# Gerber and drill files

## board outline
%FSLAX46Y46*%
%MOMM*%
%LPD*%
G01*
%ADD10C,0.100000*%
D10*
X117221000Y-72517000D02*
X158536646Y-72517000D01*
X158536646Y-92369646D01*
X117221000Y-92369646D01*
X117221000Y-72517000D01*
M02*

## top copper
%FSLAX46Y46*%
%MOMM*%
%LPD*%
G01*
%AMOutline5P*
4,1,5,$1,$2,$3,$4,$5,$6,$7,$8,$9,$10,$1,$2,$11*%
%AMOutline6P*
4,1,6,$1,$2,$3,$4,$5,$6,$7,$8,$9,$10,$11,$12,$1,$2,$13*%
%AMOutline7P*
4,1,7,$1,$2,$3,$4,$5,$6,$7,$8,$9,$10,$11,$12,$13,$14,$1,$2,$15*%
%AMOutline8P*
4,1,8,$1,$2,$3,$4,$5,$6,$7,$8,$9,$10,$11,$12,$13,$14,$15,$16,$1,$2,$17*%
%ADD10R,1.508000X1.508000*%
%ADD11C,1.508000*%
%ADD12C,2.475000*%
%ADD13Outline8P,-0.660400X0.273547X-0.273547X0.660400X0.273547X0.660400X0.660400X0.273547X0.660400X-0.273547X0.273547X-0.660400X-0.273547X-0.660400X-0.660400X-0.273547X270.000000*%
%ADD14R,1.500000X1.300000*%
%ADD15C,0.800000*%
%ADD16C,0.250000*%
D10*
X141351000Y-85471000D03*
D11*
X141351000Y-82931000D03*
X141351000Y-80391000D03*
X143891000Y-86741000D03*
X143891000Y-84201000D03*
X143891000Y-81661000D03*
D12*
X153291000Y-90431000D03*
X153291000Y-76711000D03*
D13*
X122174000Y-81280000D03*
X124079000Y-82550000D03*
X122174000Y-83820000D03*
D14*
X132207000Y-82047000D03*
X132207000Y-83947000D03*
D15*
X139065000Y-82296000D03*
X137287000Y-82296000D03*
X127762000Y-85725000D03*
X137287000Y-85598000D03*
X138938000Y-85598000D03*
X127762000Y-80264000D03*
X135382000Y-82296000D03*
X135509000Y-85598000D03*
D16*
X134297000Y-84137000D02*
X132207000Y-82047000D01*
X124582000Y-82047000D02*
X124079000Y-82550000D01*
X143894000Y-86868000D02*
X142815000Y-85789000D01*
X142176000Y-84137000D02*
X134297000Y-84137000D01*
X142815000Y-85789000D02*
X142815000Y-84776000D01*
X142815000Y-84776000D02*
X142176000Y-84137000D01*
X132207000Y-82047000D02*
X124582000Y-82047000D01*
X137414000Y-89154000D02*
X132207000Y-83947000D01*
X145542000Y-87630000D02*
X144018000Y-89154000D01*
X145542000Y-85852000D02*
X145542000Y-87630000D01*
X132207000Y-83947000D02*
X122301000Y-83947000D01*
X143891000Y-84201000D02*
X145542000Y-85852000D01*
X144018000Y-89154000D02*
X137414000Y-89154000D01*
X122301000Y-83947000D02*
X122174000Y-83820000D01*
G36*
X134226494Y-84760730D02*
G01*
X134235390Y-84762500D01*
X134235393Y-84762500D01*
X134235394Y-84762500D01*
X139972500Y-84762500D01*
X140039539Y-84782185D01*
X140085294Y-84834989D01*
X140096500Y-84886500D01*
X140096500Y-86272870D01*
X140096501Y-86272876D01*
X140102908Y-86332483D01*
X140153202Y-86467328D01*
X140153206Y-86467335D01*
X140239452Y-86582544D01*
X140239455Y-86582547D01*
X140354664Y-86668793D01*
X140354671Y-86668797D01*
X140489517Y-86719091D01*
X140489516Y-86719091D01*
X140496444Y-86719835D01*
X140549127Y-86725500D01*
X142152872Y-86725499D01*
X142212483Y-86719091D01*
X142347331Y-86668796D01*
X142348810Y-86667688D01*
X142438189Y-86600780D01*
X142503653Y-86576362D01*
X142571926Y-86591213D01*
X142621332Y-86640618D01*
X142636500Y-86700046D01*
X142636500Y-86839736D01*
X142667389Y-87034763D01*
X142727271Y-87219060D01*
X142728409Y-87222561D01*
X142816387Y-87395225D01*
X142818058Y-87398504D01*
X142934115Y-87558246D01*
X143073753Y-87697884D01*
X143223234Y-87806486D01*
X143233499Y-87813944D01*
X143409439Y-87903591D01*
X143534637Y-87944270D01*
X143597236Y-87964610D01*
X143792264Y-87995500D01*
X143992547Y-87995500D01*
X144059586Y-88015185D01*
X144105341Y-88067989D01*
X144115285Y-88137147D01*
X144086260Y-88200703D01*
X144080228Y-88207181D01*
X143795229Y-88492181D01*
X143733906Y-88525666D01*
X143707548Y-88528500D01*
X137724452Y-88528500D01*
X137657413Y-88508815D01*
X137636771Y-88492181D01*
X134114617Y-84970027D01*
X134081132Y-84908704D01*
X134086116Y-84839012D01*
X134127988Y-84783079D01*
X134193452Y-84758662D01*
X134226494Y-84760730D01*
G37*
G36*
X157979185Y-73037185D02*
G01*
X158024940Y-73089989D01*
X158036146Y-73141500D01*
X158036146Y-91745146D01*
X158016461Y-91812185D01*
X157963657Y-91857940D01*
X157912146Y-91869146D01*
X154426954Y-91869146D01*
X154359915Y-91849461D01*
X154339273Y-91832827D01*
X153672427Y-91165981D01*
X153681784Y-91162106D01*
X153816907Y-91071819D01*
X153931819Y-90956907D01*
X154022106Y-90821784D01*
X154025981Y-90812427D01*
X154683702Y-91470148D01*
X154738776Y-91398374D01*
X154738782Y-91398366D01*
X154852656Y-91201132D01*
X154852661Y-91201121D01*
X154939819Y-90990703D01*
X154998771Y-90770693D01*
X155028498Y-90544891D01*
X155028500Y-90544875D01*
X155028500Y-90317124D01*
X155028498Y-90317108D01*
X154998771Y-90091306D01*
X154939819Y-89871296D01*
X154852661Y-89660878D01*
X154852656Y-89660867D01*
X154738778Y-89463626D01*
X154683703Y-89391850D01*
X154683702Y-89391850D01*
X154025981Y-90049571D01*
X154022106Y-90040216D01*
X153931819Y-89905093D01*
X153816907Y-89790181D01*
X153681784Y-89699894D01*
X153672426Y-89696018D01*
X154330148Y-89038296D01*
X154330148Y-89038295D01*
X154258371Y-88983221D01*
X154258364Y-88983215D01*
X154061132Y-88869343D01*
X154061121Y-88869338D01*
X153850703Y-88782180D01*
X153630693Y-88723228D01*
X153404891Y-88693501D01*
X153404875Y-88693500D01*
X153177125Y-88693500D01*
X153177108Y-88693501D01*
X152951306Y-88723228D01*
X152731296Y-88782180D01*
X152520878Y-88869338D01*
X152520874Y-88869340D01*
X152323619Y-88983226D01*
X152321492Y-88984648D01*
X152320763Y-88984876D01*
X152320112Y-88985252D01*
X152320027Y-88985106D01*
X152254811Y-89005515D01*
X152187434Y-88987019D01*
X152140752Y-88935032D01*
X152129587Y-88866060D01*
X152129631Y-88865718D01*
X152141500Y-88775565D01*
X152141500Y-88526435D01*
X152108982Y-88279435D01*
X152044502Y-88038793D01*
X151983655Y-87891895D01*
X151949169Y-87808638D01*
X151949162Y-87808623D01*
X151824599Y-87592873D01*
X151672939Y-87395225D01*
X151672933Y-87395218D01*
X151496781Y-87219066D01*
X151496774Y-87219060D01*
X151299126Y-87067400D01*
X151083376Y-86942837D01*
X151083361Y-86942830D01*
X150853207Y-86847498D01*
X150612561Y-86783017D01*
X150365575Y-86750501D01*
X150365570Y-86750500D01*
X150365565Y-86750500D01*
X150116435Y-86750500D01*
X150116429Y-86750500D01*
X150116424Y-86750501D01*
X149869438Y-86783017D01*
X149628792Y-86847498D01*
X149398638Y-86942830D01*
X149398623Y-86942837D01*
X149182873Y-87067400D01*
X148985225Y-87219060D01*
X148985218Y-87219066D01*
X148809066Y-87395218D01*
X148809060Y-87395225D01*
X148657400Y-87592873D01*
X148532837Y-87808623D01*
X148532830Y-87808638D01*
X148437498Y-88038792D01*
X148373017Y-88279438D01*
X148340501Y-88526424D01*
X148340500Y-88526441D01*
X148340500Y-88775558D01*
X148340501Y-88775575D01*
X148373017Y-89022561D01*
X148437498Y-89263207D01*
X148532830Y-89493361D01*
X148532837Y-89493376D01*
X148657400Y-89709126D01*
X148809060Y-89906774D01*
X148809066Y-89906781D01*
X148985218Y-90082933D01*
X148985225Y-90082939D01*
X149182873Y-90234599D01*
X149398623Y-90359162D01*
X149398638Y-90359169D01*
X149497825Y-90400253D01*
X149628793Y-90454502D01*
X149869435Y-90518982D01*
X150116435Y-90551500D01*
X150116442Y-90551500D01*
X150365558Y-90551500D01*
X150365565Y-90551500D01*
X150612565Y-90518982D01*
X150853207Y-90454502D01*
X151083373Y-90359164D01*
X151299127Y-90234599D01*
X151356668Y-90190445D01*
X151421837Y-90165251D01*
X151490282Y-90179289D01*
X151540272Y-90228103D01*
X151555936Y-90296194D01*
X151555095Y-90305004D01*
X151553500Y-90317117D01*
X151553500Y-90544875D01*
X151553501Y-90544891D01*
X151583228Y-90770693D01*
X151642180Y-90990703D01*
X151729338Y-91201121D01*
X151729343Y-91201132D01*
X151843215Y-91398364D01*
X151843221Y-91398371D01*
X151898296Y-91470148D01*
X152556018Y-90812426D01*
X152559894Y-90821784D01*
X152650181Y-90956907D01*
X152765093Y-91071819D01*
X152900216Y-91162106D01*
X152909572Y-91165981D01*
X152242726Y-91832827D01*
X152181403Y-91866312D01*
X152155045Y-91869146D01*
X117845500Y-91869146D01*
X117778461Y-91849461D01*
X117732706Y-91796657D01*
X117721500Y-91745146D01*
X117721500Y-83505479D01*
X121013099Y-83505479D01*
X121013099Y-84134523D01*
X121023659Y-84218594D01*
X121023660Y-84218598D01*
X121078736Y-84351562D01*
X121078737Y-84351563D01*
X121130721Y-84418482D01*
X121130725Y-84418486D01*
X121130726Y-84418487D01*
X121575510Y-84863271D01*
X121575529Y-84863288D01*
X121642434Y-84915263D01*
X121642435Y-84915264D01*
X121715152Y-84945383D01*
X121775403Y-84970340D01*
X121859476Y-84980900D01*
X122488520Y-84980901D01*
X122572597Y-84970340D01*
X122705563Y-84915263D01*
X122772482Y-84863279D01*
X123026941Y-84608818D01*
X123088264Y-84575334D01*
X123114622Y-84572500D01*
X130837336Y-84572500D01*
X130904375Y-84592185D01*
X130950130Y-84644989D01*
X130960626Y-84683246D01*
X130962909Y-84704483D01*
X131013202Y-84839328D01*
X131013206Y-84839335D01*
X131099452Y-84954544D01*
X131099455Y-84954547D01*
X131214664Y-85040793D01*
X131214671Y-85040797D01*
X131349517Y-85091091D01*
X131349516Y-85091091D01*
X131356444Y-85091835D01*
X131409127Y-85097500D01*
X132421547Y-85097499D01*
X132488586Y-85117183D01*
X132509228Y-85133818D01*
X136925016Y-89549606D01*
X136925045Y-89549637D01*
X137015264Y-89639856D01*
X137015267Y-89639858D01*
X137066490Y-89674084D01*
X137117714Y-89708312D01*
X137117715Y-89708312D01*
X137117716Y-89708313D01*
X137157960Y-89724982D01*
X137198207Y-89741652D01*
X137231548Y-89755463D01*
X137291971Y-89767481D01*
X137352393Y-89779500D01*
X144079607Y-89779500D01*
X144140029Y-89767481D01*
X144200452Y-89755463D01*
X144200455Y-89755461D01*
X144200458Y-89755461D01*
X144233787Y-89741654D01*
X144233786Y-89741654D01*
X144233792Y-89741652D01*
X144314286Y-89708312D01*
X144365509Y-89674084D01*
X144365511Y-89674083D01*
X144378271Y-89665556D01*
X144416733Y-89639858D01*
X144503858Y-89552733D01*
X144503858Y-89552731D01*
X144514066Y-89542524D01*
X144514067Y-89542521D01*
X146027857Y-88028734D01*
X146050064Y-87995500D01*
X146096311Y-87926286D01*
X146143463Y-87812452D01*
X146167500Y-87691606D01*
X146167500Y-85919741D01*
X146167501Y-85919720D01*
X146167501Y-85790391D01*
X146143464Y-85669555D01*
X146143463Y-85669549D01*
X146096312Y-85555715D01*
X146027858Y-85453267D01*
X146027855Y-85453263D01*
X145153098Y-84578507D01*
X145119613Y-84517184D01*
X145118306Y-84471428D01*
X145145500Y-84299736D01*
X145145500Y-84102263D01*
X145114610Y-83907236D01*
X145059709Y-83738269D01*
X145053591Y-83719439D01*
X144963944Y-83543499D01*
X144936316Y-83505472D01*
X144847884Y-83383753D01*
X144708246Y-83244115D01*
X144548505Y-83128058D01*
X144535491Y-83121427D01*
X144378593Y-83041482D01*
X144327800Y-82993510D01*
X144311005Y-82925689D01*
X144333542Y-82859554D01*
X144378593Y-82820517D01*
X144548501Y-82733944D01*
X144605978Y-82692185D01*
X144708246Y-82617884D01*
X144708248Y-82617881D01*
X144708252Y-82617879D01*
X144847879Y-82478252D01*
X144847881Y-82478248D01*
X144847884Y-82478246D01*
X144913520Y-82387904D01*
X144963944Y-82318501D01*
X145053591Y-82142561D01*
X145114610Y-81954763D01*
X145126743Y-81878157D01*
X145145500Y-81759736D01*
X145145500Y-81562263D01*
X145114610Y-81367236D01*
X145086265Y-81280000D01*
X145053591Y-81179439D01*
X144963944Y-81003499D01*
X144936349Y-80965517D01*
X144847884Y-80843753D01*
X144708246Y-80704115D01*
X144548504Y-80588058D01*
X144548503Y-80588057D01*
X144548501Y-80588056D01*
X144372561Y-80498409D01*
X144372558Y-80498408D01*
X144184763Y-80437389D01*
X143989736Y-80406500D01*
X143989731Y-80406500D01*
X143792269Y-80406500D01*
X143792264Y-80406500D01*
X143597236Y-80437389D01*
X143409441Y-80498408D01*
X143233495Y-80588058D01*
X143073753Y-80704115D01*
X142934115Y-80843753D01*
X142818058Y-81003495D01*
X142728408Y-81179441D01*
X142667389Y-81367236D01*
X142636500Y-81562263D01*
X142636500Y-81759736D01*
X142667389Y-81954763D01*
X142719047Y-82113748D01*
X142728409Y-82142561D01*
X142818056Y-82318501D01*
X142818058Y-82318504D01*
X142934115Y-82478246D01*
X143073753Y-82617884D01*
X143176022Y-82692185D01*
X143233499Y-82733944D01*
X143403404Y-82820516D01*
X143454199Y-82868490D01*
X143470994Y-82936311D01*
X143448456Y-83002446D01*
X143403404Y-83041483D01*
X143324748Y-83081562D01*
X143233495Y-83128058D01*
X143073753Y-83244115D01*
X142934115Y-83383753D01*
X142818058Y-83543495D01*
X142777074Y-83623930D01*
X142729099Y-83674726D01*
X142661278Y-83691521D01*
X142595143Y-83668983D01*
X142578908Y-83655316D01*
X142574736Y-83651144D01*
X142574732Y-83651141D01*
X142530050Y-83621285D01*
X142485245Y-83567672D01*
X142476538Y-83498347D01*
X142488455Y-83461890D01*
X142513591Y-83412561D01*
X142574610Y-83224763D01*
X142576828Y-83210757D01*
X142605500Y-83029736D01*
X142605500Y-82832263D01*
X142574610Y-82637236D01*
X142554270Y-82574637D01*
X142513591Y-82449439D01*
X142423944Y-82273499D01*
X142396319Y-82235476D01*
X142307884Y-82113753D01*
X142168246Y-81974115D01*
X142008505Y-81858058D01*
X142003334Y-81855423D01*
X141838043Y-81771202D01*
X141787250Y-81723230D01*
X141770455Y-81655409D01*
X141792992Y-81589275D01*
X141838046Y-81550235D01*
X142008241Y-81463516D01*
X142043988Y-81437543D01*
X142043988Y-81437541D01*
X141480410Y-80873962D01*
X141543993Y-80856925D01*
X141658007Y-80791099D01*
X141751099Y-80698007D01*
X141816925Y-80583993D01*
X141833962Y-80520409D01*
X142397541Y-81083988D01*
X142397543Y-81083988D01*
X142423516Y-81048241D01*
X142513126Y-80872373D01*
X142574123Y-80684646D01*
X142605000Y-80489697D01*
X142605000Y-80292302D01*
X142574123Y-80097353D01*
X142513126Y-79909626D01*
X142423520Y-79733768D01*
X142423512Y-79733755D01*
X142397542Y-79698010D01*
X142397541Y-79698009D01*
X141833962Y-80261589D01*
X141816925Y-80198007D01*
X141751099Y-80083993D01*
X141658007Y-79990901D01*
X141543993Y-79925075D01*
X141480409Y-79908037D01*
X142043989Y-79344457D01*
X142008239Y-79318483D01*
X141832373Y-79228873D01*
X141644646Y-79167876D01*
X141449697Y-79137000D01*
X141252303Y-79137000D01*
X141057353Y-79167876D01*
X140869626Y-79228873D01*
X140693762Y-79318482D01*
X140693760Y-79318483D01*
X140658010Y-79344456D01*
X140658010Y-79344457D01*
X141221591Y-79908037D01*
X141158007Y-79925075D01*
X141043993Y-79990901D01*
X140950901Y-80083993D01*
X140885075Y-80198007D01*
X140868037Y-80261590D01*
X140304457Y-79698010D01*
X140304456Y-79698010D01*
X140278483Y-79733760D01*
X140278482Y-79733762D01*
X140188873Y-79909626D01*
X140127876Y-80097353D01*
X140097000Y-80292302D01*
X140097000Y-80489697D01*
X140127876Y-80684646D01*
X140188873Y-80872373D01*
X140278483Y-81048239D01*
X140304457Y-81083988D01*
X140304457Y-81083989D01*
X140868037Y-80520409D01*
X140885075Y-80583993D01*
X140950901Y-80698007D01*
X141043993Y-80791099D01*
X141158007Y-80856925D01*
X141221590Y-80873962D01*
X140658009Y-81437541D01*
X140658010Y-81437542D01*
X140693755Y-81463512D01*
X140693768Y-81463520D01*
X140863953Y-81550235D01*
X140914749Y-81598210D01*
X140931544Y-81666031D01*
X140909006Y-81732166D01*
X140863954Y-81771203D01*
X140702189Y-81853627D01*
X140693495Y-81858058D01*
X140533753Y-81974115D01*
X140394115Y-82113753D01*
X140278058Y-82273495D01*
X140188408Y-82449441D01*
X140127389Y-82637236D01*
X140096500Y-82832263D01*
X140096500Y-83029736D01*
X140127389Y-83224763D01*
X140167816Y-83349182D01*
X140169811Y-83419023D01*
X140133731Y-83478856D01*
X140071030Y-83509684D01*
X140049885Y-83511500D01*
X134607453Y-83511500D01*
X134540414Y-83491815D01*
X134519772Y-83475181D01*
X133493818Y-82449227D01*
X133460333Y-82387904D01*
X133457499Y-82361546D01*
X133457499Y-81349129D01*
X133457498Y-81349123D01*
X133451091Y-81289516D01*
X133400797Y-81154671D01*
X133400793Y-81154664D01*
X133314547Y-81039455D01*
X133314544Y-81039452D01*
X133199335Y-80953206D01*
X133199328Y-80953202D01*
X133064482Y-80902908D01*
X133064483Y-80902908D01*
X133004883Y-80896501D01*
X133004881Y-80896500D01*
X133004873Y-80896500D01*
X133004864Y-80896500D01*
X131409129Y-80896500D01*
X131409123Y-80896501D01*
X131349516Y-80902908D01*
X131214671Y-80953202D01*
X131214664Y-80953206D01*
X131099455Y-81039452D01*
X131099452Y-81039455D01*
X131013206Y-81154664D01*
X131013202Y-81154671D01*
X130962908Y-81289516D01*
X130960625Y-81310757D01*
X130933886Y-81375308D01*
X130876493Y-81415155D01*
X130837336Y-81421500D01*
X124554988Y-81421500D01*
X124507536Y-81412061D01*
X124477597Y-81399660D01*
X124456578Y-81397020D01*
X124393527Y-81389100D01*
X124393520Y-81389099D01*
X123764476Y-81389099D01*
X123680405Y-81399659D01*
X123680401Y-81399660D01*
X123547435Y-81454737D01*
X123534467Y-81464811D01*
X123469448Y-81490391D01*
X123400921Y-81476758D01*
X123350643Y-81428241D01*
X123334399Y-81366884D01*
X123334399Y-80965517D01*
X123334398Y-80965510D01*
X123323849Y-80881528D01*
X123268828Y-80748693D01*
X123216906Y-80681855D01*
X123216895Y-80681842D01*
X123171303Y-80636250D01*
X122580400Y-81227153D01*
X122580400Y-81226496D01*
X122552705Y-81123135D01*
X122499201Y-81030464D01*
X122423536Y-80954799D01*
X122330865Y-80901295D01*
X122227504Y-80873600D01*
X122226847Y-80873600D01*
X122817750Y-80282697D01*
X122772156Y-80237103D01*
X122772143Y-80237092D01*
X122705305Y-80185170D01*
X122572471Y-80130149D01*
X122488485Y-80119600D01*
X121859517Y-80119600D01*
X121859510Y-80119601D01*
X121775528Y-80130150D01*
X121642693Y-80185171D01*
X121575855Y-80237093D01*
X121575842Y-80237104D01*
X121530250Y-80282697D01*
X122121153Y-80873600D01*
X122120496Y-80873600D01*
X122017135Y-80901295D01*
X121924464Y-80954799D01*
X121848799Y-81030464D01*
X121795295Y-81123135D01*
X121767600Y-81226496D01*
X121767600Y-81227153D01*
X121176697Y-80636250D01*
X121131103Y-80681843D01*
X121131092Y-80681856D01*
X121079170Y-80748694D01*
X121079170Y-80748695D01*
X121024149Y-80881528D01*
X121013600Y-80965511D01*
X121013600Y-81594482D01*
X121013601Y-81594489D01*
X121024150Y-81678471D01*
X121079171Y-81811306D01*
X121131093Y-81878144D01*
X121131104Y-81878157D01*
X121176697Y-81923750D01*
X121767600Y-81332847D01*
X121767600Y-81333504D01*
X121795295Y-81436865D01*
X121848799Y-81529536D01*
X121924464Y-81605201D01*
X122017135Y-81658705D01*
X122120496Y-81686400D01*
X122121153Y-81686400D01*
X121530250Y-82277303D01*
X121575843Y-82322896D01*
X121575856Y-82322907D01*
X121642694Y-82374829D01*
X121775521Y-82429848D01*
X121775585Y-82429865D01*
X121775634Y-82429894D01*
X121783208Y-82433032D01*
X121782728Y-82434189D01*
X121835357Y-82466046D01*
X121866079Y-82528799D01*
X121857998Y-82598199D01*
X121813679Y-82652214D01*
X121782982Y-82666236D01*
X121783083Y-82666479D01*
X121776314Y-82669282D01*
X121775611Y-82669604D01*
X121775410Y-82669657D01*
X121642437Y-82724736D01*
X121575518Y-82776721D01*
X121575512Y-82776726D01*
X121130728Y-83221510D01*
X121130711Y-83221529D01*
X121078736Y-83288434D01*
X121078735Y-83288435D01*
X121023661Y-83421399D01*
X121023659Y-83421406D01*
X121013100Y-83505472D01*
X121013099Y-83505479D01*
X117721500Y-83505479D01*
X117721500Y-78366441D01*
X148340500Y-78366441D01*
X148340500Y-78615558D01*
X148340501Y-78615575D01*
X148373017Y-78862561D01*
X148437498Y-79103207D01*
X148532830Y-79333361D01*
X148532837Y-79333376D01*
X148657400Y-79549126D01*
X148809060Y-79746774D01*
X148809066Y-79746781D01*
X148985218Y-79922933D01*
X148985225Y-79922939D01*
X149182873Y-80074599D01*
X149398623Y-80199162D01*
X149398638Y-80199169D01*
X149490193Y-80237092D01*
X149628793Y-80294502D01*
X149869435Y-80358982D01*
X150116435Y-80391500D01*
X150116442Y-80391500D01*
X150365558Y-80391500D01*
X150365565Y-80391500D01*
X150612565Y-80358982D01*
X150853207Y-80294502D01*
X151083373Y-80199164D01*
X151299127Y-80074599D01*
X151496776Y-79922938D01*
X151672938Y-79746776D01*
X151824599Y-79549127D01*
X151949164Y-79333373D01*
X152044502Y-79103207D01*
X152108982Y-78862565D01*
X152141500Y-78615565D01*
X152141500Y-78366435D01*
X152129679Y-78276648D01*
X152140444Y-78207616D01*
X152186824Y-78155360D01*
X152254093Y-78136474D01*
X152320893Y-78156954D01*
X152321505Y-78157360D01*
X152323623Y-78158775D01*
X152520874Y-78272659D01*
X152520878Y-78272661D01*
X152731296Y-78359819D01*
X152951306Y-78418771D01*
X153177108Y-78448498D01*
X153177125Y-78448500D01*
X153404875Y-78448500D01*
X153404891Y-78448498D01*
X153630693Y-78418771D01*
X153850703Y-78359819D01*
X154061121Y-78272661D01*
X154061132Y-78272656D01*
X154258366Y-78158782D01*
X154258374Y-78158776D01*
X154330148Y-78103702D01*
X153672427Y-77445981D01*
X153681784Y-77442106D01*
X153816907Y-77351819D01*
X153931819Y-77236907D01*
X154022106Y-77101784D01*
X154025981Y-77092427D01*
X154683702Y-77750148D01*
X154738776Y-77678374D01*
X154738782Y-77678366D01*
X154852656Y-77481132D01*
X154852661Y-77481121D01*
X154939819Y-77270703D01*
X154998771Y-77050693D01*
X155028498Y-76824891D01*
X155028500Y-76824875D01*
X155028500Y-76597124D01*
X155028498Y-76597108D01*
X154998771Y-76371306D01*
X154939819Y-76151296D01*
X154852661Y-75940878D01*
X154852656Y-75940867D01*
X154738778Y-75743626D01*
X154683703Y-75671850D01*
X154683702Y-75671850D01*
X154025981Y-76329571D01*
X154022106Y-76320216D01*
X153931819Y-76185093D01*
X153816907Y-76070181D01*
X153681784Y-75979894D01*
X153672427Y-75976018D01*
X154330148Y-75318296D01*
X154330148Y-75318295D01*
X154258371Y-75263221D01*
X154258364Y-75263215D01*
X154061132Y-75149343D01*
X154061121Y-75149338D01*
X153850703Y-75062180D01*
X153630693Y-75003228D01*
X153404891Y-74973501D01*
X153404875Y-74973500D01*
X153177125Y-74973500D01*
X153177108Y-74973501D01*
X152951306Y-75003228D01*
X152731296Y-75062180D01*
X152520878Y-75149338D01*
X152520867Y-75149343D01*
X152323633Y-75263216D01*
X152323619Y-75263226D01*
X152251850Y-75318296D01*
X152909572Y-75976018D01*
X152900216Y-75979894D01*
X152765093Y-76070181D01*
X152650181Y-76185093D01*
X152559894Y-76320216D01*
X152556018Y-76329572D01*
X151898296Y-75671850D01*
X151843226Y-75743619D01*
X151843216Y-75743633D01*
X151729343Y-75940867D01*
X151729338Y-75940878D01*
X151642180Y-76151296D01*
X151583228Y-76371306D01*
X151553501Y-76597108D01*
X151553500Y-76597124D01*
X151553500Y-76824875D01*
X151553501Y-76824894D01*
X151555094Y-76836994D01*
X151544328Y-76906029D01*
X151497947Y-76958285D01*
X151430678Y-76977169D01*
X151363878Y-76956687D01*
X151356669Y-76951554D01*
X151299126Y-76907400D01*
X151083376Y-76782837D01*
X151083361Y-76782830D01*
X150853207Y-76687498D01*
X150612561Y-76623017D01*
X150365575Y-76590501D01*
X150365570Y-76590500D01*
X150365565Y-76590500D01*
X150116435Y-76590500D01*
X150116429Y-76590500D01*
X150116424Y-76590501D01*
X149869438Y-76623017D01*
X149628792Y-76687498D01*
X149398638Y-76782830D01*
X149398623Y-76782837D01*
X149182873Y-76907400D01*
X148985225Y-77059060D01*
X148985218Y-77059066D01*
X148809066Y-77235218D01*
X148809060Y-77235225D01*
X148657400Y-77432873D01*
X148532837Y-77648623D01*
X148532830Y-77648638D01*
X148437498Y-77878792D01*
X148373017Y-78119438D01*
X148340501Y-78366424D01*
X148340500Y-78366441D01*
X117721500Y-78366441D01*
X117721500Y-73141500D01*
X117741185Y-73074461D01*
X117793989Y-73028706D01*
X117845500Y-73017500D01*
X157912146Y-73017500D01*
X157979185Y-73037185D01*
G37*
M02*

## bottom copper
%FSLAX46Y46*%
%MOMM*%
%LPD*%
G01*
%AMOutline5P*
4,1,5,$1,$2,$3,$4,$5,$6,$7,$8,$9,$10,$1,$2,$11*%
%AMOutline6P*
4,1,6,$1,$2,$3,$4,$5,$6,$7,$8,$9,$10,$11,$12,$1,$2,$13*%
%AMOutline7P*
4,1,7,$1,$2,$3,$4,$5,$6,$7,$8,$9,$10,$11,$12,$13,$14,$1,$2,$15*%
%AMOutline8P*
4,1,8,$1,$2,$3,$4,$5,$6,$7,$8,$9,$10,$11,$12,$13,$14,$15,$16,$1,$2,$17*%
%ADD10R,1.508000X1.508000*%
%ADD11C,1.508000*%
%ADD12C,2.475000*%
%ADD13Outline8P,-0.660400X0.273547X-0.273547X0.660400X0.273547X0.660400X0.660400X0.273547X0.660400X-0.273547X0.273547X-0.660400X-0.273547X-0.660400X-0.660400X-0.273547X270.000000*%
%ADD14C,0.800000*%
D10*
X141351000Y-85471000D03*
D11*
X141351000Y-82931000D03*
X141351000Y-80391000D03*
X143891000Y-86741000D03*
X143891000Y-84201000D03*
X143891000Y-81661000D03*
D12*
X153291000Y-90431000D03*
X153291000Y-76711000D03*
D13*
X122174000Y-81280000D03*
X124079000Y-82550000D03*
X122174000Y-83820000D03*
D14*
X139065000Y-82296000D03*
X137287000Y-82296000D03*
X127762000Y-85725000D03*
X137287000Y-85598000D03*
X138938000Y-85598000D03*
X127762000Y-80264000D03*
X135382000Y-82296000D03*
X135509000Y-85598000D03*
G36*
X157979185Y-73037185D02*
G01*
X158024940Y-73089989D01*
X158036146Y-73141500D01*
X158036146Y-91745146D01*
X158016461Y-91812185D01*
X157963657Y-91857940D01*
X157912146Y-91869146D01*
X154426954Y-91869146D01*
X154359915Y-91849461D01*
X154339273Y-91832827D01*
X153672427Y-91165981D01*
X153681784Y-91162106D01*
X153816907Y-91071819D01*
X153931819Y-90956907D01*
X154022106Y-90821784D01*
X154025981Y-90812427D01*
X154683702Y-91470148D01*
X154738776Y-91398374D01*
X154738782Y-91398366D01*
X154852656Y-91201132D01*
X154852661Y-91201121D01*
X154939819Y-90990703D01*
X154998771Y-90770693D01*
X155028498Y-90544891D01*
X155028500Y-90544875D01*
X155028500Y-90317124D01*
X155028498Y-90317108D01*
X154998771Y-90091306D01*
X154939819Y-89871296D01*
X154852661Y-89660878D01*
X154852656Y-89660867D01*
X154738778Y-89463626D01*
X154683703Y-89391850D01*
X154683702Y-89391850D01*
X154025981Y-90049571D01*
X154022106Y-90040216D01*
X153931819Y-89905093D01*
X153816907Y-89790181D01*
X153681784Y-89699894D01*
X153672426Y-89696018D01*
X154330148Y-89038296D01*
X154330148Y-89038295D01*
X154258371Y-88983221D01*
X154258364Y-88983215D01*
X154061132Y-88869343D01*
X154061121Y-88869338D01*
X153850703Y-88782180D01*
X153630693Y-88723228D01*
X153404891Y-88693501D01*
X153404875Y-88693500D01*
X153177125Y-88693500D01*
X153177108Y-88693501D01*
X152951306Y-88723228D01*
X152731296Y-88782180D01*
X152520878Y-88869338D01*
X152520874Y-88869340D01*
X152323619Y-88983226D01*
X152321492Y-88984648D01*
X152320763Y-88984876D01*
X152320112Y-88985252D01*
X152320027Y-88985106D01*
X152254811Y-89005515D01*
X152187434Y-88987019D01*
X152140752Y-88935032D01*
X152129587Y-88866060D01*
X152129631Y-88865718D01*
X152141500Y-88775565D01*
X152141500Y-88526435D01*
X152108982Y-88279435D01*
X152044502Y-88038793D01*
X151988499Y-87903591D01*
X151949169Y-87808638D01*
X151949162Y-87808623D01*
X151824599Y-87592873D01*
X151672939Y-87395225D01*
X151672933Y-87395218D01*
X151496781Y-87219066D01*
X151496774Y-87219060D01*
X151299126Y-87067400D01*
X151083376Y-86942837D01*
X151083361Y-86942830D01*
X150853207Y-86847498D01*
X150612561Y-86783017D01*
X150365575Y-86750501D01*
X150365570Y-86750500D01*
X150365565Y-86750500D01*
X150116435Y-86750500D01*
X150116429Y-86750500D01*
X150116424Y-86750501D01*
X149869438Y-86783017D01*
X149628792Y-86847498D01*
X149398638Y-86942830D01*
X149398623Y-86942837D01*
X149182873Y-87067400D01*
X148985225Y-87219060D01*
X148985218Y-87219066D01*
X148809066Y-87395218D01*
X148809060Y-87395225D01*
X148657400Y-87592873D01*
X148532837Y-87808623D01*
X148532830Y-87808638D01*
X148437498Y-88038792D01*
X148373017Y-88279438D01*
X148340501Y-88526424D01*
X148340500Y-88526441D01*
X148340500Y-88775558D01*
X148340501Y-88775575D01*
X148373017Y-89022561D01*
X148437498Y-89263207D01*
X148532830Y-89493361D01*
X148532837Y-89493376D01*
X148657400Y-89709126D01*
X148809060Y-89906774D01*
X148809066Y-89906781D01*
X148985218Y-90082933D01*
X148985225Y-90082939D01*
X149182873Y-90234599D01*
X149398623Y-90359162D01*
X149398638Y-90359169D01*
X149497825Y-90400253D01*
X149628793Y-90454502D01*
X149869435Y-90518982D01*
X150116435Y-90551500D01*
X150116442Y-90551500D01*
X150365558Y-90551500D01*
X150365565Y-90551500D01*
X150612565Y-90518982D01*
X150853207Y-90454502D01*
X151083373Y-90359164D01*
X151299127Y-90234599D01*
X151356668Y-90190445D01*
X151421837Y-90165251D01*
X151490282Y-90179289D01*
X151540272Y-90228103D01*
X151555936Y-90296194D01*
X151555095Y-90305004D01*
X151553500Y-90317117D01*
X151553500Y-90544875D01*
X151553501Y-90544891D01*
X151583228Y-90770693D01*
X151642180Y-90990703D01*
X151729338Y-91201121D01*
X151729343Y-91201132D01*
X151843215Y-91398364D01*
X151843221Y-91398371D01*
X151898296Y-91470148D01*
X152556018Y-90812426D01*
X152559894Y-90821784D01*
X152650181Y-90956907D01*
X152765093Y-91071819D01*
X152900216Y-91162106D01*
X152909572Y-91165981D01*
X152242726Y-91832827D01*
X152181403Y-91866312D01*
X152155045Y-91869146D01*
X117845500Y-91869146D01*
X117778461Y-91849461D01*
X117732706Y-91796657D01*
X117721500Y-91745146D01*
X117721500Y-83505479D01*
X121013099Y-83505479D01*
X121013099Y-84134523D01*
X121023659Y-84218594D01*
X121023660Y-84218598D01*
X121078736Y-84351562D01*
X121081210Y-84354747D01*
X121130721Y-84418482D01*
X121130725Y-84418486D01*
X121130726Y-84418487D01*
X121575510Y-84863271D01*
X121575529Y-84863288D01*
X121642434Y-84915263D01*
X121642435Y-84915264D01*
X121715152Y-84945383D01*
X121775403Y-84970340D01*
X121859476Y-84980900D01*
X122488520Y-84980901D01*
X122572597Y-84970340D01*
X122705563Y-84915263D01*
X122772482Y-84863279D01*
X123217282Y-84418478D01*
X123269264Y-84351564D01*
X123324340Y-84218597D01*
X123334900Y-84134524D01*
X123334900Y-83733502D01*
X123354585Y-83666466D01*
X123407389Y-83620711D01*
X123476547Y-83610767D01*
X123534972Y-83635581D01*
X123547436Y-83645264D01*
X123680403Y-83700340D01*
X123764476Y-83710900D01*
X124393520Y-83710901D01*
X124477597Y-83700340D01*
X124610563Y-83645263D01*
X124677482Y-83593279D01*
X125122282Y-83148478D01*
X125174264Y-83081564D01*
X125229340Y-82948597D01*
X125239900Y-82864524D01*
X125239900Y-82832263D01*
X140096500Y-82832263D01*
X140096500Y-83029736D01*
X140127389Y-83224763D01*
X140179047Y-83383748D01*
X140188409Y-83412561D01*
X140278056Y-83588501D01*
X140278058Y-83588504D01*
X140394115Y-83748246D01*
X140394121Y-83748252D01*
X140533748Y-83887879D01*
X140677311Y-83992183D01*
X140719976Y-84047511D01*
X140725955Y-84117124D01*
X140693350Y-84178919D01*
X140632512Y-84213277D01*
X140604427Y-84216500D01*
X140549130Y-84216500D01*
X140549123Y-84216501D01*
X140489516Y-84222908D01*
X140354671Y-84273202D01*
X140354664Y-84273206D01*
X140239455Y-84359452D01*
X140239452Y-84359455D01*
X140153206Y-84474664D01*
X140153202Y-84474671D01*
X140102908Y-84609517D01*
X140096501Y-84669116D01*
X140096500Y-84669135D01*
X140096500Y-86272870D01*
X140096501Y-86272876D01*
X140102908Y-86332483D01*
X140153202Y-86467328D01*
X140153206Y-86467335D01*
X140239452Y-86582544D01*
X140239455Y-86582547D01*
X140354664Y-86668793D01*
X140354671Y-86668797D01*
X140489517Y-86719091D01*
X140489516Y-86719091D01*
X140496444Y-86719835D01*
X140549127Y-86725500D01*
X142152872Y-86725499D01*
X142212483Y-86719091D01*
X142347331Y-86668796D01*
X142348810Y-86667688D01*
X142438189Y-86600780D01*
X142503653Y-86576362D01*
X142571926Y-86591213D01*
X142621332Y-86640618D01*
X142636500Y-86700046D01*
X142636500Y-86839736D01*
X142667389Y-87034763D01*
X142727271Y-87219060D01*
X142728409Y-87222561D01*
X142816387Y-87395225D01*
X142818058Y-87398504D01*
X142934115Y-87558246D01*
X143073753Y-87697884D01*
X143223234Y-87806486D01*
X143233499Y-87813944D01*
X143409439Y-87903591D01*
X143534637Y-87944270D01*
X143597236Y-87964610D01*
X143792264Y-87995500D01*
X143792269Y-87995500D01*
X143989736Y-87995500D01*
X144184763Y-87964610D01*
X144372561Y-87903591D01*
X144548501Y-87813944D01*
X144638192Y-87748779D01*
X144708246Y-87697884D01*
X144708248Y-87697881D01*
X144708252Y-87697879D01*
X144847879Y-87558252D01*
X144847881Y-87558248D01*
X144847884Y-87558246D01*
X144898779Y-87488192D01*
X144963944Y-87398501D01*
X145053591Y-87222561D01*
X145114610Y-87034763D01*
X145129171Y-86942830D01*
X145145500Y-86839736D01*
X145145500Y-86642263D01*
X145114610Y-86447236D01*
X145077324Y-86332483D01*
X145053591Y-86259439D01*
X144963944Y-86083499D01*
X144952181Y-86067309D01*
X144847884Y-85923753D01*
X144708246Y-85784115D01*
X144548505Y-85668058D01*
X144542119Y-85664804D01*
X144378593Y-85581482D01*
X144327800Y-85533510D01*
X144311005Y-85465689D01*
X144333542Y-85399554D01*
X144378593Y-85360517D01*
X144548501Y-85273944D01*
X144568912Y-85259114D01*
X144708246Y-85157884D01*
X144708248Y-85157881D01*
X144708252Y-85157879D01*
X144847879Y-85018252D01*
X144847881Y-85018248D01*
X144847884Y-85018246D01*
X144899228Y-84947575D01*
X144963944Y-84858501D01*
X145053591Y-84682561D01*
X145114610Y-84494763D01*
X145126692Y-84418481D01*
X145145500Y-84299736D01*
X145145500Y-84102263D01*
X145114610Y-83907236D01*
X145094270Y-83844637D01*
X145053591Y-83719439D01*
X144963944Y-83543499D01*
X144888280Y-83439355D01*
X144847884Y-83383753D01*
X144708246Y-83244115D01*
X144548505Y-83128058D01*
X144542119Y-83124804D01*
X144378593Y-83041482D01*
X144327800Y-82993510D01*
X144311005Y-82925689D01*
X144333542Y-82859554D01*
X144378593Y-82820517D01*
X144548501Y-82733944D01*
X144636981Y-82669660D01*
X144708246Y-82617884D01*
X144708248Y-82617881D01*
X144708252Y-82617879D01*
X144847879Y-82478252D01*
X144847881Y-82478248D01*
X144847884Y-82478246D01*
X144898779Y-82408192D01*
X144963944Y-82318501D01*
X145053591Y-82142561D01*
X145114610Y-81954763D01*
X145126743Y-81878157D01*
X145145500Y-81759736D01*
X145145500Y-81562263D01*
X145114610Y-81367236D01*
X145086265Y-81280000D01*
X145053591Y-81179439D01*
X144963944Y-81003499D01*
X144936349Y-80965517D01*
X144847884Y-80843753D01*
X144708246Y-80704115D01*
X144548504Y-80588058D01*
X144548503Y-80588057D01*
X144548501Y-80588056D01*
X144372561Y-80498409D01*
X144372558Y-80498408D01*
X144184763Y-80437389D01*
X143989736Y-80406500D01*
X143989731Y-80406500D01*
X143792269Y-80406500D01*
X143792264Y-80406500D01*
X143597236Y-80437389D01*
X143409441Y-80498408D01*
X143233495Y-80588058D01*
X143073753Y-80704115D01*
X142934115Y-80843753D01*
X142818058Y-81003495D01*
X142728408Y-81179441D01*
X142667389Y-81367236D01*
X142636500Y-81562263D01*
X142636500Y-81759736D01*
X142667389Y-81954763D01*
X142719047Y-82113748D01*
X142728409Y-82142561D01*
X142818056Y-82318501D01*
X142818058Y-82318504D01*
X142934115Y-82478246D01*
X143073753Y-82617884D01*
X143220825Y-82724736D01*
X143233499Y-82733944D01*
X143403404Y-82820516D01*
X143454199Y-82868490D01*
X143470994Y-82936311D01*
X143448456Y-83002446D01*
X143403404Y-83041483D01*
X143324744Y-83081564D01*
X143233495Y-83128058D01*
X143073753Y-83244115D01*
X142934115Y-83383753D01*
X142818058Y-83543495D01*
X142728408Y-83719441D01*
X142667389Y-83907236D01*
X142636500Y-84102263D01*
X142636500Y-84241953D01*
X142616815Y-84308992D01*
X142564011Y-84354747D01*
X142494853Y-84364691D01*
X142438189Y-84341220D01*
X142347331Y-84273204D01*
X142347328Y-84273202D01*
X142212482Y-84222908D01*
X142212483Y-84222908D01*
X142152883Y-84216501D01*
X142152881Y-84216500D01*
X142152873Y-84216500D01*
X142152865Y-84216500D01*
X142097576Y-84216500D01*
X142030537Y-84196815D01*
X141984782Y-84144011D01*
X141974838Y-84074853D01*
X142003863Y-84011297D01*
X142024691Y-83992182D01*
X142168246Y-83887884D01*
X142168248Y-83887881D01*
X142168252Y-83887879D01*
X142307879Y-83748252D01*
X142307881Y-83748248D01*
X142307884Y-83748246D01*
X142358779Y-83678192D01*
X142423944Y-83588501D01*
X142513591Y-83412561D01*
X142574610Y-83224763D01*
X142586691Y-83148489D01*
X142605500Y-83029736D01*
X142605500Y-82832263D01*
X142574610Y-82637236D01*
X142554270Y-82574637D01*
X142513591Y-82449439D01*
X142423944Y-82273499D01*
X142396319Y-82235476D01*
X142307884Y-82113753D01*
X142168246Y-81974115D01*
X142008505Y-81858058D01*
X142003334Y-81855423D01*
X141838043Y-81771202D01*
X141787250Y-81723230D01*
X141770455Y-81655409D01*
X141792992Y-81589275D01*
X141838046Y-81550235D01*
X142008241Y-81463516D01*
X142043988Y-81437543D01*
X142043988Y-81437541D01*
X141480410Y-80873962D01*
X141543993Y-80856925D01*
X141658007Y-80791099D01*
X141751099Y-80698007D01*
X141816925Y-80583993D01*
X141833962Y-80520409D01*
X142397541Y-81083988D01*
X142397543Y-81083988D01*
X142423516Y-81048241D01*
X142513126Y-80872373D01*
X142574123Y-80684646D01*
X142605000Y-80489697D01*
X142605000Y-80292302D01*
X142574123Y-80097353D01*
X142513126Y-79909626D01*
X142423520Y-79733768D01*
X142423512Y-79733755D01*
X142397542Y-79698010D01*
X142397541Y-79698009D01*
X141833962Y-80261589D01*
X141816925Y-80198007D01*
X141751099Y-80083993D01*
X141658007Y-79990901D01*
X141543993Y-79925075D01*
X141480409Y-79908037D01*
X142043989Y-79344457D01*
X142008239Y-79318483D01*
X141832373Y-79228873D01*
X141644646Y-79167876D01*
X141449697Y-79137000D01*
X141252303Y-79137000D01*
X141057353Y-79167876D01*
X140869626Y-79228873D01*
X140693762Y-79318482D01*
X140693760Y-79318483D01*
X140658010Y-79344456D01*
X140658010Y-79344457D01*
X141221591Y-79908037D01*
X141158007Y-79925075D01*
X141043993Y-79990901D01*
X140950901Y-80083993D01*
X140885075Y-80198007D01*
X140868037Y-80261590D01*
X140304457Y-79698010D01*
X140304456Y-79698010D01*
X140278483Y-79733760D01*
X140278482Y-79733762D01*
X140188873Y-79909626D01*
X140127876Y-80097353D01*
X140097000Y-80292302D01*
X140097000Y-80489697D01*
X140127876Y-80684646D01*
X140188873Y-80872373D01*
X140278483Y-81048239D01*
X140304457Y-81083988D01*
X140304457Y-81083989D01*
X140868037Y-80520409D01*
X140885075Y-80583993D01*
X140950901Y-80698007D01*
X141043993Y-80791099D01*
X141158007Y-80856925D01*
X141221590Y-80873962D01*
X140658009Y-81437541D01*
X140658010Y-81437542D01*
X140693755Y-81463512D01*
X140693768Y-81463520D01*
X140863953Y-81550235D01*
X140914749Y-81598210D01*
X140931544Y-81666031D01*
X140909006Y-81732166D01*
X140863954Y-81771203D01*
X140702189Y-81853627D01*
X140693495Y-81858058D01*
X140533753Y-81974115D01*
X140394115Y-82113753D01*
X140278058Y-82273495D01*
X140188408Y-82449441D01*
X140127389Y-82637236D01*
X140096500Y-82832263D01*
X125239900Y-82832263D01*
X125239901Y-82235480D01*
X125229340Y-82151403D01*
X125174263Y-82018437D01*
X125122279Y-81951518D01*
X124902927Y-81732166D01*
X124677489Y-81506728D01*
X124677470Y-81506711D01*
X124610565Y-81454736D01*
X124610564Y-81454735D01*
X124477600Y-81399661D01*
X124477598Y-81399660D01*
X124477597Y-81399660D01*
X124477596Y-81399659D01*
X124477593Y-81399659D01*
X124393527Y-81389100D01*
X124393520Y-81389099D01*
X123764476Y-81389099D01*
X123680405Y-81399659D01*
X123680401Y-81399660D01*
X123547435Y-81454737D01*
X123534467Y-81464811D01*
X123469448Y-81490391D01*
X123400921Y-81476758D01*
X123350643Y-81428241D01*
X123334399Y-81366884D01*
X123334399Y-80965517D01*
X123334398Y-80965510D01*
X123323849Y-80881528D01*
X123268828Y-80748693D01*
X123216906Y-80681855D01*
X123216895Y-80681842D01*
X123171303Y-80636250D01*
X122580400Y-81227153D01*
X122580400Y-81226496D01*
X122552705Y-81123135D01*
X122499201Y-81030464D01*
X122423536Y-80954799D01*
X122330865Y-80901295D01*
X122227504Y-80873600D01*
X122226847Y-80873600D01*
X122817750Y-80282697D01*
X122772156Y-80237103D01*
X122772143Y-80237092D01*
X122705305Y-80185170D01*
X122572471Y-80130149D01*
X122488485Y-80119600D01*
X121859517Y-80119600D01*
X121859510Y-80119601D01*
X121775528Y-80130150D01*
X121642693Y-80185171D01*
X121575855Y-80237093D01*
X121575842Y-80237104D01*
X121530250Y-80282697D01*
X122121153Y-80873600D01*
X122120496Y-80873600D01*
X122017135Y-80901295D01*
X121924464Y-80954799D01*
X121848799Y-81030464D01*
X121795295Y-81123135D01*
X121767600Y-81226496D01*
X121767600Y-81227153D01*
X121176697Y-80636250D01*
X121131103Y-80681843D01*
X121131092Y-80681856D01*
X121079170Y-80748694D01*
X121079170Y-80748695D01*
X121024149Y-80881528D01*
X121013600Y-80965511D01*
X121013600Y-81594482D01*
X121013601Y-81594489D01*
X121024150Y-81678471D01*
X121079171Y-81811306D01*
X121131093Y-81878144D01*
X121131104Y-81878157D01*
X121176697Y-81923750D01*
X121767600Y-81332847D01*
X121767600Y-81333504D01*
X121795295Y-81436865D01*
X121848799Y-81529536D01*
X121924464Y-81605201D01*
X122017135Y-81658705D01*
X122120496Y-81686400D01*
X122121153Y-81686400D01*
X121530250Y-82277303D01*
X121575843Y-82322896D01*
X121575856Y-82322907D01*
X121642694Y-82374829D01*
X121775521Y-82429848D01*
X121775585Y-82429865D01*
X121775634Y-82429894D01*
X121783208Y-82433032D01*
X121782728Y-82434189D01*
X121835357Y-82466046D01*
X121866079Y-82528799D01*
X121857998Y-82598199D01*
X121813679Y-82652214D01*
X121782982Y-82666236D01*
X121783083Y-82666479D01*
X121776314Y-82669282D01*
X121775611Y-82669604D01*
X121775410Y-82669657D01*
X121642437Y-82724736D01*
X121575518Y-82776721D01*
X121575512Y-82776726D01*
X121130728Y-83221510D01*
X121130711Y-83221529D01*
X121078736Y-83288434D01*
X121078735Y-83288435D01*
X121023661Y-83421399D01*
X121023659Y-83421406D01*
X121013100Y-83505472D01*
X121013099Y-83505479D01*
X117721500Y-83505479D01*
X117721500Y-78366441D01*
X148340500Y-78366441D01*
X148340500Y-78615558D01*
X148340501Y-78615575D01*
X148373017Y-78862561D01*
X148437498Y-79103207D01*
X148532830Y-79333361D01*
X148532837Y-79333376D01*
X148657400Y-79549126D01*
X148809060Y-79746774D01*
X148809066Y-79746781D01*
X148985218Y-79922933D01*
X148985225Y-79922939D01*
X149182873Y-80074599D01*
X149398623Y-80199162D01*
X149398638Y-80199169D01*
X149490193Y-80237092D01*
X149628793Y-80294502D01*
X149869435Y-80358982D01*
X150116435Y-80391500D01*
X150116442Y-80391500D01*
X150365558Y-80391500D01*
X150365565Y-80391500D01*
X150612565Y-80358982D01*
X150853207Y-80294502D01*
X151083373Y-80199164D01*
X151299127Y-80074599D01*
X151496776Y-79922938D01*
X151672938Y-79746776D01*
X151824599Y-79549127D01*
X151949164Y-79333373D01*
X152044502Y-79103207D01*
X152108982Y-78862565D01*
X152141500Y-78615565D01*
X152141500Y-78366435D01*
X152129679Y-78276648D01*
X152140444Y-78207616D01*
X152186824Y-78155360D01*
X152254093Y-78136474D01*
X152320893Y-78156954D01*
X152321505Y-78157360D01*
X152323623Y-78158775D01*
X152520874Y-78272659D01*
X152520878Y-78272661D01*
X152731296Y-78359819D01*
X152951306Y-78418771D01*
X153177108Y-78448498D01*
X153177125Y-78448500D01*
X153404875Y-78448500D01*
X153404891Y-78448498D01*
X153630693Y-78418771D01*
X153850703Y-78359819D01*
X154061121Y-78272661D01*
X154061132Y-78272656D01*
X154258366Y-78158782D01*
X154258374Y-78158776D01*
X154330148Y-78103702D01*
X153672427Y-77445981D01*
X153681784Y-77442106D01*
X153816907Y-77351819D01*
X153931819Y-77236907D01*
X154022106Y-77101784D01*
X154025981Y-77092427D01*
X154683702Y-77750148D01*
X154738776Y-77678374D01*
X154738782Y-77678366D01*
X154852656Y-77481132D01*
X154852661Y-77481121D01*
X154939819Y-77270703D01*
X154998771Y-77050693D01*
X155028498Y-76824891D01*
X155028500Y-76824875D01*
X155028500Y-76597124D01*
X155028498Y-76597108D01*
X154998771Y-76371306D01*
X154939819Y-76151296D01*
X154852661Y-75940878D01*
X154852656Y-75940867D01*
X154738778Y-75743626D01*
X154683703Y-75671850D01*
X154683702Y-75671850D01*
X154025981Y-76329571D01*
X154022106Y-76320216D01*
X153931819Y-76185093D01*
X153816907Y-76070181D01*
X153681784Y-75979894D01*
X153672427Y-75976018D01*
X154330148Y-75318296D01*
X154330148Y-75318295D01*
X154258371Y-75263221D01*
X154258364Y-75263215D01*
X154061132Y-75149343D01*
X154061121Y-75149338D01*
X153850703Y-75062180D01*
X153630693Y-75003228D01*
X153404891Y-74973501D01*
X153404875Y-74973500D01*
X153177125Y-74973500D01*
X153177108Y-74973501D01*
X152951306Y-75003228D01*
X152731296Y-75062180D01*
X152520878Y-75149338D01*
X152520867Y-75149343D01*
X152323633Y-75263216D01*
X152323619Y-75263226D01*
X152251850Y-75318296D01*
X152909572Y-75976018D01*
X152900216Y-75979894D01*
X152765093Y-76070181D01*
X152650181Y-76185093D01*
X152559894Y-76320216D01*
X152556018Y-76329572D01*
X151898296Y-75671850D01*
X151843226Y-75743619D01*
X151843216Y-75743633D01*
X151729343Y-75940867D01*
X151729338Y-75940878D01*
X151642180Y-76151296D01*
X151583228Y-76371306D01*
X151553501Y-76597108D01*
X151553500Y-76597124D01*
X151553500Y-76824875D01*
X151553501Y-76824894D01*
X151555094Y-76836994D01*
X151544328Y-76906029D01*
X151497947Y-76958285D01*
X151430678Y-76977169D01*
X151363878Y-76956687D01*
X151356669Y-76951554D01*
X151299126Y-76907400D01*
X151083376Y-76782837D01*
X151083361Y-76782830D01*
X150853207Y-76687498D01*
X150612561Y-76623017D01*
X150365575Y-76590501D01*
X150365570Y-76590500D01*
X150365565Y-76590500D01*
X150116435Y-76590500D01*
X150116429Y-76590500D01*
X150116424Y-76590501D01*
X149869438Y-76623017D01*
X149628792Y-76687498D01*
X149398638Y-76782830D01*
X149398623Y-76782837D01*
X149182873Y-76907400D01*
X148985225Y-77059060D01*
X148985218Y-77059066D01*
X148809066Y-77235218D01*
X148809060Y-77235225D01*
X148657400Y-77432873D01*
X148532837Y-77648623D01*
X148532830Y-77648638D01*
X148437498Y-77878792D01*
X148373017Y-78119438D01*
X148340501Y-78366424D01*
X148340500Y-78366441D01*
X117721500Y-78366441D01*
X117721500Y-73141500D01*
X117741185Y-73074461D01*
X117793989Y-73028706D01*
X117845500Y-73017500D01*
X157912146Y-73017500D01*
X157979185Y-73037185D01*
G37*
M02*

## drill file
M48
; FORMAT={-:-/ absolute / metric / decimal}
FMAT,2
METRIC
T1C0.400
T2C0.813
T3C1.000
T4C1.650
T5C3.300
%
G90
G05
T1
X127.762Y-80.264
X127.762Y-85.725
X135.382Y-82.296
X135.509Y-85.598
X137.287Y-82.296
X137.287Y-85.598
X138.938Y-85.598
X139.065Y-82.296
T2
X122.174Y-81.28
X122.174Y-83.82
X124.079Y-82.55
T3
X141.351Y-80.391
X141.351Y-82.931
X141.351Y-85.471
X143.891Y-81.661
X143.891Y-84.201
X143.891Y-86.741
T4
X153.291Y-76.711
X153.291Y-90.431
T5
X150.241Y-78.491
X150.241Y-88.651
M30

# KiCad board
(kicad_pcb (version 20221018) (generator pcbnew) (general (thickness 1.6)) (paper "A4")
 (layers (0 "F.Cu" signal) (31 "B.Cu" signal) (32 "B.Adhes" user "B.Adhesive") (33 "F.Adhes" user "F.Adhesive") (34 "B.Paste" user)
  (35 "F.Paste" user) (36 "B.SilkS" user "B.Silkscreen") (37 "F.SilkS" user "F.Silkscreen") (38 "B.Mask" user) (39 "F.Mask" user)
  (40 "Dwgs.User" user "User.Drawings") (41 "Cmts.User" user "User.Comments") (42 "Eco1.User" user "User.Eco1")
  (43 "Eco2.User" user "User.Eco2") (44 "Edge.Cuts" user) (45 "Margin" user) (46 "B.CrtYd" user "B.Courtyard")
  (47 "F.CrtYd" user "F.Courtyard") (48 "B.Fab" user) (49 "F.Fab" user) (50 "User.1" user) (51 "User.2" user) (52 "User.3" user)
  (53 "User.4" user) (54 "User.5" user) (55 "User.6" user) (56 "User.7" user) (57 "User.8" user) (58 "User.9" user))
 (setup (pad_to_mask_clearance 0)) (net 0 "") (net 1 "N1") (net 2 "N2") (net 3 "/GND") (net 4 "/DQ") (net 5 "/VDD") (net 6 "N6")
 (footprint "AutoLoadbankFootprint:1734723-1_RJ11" (layer "F.Cu") (at 143.891 82.931 90)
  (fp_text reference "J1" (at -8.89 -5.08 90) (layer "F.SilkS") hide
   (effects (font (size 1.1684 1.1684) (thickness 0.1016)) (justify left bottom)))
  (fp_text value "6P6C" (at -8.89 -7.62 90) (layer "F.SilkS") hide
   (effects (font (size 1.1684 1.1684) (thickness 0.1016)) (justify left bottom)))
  (pad "" np_thru_hole circle (at -5.72 6.35 90) (size 3.3 3.3) (drill 3.3) (layers "*.Cu" "*.Mask"))
  (pad "" np_thru_hole circle (at 4.44 6.35 90) (size 3.3 3.3) (drill 3.3) (layers "*.Cu" "*.Mask"))
  (pad "1" thru_hole rect (at -2.54 -2.54 90) (size 1.508 1.508) (drill 1) (layers "*.Cu" "*.Mask") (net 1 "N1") (solder_mask_margin 0.1016)
   (thermal_bridge_angle 45))
  (pad "2" thru_hole circle (at 0 -2.54 90) (size 1.508 1.508) (drill 1) (layers "*.Cu" "*.Mask") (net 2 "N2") (solder_mask_margin 0.1016))
  (pad "3" thru_hole circle (at 2.54 -2.54 90) (size 1.508 1.508) (drill 1) (layers "*.Cu" "*.Mask") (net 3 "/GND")
   (solder_mask_margin 0.1016))
  (pad "4" thru_hole circle (at -3.81 0 90) (size 1.508 1.508) (drill 1) (layers "*.Cu" "*.Mask") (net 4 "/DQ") (solder_mask_margin 0.1016))
  (pad "5" thru_hole circle (at -1.27 0 90) (size 1.508 1.508) (drill 1) (layers "*.Cu" "*.Mask") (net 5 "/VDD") (solder_mask_margin 0.1016))
  (pad "6" thru_hole circle (at 1.27 0 90) (size 1.508 1.508) (drill 1) (layers "*.Cu" "*.Mask") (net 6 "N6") (solder_mask_margin 0.1016))
  (pad "SH1" thru_hole circle (at -7.5 9.4 90) (size 2.475 2.475) (drill 1.65) (layers "*.Cu" "*.Mask") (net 3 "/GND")
   (solder_mask_margin 0.1016))
  (pad "SH2" thru_hole circle (at 6.22 9.4 90) (size 2.475 2.475) (drill 1.65) (layers "*.Cu" "*.Mask") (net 3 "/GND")
   (solder_mask_margin 0.1016)))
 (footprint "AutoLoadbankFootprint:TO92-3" (layer "F.Cu") (at 122.174 82.55 -90)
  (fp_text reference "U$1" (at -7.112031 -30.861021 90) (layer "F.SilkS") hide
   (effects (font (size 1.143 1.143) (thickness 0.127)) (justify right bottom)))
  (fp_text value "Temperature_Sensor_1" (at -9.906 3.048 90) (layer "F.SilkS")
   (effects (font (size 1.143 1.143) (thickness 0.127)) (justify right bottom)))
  (pad "1" thru_hole roundrect (at -1.27 0 270) (size 1.3208 1.3208) (drill 0.8128) (layers "*.Cu" "*.Mask") (roundrect_rratio 0.25)
   (chamfer_ratio 0.2928932188) (chamfer top_left top_right bottom_left bottom_right) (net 3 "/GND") (solder_mask_margin 0.1016)
   (thermal_bridge_angle 45))
  (pad "2" thru_hole roundrect (at 0 -1.905 270) (size 1.3208 1.3208) (drill 0.8128) (layers "*.Cu" "*.Mask") (roundrect_rratio 0.25)
   (chamfer_ratio 0.2928932188) (chamfer top_left top_right bottom_left bottom_right) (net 4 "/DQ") (solder_mask_margin 0.1016)
   (thermal_bridge_angle 45))
  (pad "3" thru_hole roundrect (at 1.27 0 270) (size 1.3208 1.3208) (drill 0.8128) (layers "*.Cu" "*.Mask") (roundrect_rratio 0.25)
   (chamfer_ratio 0.2928932188) (chamfer top_left top_right bottom_left bottom_right) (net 5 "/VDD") (solder_mask_margin 0.1016)
   (thermal_bridge_angle 45)))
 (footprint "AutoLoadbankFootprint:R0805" (layer "F.Cu") (at 132.207 82.997 -90)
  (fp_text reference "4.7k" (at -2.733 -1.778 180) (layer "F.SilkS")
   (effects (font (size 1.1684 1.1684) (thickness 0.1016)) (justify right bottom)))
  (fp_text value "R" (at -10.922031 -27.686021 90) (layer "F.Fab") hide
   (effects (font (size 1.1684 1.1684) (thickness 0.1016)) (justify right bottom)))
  (pad "1" smd rect (at -0.95 0 270) (size 1.3 1.5) (layers "F.Cu" "F.Paste" "F.Mask") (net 4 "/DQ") (solder_mask_margin 0.1016)
   (thermal_bridge_angle 45))
  (pad "2" smd rect (at 0.95 0 270) (size 1.3 1.5) (layers "F.Cu" "F.Paste" "F.Mask") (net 5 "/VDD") (solder_mask_margin 0.1016)
   (thermal_bridge_angle 45)))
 (gr_rect (start 117.221 72.517) (end 158.536646 92.369646) (stroke (width 0.1) (type default)) (fill none) (layer "Edge.Cuts"))
 (segment (start 134.297 84.137) (end 132.207 82.047) (width 0.25) (layer "F.Cu") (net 4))
 (segment (start 124.582 82.047) (end 124.079 82.55) (width 0.25) (layer "F.Cu") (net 4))
 (segment (start 143.894 86.868) (end 142.815 85.789) (width 0.25) (layer "F.Cu") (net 4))
 (segment (start 142.176 84.137) (end 134.297 84.137) (width 0.25) (layer "F.Cu") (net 4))
 (segment (start 142.815 85.789) (end 142.815 84.776) (width 0.25) (layer "F.Cu") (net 4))
 (segment (start 142.815 84.776) (end 142.176 84.137) (width 0.25) (layer "F.Cu") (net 4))
 (segment (start 132.207 82.047) (end 124.582 82.047) (width 0.25) (layer "F.Cu") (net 4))
 (segment (start 137.414 89.154) (end 132.207 83.947) (width 0.25) (layer "F.Cu") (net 5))
 (segment (start 145.542 87.63) (end 144.018 89.154) (width 0.25) (layer "F.Cu") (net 5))
 (segment (start 145.542 85.852) (end 145.542 87.63) (width 0.25) (layer "F.Cu") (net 5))
 (segment (start 132.207 83.947) (end 122.301 83.947) (width 0.25) (layer "F.Cu") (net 5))
 (segment (start 143.891 84.201) (end 145.542 85.852) (width 0.25) (layer "F.Cu") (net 5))
 (segment (start 144.018 89.154) (end 137.414 89.154) (width 0.25) (layer "F.Cu") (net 5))
 (segment (start 122.301 83.947) (end 122.174 83.82) (width 0.25) (layer "F.Cu") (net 5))
 (via (at 139.065 82.296) (size 0.8) (drill 0.4) (layers "F.Cu" "B.Cu") (free) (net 3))
 (via (at 137.287 82.296) (size 0.8) (drill 0.4) (layers "F.Cu" "B.Cu") (free) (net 3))
 (via (at 127.762 85.725) (size 0.8) (drill 0.4) (layers "F.Cu" "B.Cu") (free) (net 3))
 (via (at 137.287 85.598) (size 0.8) (drill 0.4) (layers "F.Cu" "B.Cu") (free) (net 3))
 (via (at 138.938 85.598) (size 0.8) (drill 0.4) (layers "F.Cu" "B.Cu") (free) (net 3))
 (via (at 127.762 80.264) (size 0.8) (drill 0.4) (layers "F.Cu" "B.Cu") (free) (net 3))
 (via (at 135.382 82.296) (size 0.8) (drill 0.4) (layers "F.Cu" "B.Cu") (free) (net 3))
 (via (at 135.509 85.598) (size 0.8) (drill 0.4) (layers "F.Cu" "B.Cu") (free) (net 3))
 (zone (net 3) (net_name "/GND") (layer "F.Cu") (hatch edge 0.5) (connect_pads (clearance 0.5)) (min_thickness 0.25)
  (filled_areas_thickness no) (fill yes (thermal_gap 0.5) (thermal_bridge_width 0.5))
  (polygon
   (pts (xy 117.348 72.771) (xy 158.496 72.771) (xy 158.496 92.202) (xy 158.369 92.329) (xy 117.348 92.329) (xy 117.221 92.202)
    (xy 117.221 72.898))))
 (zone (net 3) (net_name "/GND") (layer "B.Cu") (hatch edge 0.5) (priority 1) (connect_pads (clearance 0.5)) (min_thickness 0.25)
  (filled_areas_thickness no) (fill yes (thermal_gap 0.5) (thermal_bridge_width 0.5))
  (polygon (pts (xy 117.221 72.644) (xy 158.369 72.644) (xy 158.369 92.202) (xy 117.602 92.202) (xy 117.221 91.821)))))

